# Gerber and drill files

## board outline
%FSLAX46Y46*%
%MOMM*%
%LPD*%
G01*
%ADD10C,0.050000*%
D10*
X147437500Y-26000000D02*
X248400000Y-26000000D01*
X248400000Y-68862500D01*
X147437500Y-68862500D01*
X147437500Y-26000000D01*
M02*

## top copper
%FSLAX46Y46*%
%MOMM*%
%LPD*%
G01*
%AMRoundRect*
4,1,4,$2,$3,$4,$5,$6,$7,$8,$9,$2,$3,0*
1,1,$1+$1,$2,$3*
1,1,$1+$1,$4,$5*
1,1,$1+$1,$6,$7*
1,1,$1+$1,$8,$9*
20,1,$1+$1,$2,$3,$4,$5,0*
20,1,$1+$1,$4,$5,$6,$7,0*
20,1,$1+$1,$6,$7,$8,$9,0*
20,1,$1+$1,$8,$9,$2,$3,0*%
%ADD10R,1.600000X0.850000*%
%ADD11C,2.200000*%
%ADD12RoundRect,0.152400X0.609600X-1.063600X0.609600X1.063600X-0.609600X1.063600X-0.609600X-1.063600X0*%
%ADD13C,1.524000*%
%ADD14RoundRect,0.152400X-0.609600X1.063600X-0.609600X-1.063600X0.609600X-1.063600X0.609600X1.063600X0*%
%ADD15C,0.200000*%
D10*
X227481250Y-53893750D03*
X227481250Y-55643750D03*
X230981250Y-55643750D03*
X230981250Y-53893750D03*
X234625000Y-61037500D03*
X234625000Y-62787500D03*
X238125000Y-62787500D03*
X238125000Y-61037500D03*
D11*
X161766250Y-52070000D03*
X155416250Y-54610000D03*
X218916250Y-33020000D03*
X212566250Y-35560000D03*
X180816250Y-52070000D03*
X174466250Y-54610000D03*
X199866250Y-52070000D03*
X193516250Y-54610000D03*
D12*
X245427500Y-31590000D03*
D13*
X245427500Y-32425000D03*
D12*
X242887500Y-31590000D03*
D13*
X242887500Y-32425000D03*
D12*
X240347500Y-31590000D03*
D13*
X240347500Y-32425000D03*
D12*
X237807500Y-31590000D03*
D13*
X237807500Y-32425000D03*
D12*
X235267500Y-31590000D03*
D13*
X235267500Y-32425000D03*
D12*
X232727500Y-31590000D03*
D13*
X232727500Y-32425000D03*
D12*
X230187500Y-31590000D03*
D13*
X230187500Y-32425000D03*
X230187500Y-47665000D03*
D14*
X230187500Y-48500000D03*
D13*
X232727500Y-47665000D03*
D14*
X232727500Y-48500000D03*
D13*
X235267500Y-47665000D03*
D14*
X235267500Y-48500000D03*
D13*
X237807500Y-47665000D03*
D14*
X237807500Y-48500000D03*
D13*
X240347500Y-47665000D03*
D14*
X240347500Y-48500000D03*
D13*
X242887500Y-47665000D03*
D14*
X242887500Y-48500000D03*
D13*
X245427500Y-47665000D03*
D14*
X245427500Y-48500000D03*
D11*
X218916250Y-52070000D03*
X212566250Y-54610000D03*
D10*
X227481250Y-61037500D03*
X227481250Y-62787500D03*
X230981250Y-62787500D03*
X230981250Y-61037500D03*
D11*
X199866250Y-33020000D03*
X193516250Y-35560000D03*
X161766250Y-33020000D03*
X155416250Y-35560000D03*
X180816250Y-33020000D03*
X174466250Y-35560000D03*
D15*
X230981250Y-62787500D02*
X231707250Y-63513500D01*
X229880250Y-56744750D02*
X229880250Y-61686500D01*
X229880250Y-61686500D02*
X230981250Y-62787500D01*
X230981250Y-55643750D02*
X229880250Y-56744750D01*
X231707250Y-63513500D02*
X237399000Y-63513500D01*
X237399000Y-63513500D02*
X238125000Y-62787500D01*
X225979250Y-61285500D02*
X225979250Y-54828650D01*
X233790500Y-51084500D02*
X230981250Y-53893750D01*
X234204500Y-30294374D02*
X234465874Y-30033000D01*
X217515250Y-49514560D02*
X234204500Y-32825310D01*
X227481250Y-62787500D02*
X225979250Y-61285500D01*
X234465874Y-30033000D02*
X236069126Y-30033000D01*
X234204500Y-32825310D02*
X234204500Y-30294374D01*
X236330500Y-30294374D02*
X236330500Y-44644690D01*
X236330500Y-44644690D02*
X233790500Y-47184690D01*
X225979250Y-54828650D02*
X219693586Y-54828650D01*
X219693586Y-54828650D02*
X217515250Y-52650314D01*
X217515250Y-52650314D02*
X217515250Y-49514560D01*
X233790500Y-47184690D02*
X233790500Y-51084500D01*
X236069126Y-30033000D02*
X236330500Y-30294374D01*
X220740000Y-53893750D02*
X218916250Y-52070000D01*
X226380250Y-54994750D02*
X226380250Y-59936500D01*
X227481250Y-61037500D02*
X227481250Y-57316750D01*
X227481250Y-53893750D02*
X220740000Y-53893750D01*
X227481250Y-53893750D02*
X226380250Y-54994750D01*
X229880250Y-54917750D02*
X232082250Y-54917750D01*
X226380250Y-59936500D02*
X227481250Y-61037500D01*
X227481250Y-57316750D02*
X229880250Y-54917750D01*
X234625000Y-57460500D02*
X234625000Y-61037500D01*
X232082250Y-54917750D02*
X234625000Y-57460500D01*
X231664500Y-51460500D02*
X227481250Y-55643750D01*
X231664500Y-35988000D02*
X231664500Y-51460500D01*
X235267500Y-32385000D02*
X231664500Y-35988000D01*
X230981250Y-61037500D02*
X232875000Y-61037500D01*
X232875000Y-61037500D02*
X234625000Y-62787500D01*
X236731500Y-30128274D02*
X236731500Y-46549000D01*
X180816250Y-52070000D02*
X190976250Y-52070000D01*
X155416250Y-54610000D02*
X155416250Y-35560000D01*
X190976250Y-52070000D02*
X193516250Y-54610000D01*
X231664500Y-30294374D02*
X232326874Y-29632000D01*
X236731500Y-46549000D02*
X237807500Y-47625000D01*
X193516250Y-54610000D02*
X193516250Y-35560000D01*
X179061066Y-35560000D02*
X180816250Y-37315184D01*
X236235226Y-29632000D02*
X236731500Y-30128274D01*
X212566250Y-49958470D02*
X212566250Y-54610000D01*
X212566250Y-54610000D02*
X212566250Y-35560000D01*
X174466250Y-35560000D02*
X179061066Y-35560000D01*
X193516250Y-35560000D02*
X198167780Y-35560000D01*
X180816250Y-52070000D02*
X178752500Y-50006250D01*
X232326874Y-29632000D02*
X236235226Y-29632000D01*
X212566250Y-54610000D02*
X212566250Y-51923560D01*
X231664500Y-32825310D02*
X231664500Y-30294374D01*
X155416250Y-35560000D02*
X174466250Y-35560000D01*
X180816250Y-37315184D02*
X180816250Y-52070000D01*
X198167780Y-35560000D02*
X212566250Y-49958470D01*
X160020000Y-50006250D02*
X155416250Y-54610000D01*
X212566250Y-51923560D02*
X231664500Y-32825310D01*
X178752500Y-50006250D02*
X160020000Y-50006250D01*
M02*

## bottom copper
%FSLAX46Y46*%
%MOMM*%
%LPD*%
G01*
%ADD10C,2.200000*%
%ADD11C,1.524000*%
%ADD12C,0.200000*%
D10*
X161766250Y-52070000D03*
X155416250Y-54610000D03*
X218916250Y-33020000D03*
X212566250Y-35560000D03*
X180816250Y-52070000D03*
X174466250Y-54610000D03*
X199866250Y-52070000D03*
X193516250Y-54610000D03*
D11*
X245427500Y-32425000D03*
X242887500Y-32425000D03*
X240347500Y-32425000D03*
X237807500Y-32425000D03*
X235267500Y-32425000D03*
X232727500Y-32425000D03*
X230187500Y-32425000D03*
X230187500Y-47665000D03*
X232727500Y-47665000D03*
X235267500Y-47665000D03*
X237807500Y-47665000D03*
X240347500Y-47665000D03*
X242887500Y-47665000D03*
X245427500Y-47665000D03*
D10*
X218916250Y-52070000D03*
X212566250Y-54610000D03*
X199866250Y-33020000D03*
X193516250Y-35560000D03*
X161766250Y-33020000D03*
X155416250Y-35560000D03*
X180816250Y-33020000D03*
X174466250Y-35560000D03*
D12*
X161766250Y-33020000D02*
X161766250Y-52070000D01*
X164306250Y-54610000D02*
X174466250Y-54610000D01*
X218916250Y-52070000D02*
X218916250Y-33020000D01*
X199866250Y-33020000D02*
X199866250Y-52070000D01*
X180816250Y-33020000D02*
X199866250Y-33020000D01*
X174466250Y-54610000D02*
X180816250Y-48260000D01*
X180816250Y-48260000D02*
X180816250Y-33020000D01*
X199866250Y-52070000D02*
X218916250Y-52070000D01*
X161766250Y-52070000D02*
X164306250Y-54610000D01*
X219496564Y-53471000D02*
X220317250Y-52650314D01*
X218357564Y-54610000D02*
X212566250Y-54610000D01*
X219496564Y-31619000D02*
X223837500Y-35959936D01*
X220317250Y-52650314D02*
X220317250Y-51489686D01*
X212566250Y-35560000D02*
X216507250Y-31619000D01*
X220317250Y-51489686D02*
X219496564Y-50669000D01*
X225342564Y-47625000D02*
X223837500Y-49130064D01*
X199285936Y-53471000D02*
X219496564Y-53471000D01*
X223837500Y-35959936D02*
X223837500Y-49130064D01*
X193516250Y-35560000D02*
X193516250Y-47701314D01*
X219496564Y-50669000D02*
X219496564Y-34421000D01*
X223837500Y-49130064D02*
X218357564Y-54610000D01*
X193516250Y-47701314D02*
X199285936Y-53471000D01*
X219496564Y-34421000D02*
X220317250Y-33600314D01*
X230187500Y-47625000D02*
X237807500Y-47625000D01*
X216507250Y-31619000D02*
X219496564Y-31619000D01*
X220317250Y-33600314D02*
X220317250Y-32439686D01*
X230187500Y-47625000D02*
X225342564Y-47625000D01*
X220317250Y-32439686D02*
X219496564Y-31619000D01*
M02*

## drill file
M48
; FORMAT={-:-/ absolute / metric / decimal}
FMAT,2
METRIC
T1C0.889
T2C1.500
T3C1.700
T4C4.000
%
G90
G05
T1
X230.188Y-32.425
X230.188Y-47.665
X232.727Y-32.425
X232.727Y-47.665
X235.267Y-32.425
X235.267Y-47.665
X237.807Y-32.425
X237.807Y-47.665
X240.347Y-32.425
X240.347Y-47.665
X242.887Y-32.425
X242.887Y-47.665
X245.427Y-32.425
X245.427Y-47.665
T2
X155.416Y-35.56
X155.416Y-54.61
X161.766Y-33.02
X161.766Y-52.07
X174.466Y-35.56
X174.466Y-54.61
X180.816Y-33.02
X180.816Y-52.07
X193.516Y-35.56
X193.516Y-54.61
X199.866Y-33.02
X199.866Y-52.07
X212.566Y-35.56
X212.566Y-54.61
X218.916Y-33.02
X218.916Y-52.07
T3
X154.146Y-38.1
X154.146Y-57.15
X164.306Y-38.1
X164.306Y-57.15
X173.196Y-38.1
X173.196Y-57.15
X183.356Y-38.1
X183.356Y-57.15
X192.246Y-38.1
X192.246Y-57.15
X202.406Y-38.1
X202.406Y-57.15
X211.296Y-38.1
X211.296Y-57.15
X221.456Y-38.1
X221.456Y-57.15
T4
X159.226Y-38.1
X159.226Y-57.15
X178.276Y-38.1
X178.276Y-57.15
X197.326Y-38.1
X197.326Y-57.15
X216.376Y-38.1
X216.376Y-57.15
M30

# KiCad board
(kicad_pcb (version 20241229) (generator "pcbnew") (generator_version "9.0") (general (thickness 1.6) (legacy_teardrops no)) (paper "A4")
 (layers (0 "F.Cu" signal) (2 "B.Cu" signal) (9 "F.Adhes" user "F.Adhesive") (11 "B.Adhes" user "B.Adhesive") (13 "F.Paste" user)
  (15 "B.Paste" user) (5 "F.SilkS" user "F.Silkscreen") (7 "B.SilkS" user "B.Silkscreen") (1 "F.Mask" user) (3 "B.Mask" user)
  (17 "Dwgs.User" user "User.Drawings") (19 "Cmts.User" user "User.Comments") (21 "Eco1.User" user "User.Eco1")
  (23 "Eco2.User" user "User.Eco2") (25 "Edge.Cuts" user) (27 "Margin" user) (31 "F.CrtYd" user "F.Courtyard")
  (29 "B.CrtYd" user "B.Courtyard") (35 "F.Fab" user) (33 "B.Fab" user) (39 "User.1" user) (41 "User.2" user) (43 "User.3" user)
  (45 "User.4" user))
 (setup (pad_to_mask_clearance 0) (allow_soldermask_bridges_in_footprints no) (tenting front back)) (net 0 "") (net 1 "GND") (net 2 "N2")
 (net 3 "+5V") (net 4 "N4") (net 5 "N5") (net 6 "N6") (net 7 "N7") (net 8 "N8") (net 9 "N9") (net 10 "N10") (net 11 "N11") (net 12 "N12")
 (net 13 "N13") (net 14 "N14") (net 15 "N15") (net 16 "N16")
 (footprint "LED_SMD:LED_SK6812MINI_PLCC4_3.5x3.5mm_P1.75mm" (layer "F.Cu") (at 229.23125 54.76875)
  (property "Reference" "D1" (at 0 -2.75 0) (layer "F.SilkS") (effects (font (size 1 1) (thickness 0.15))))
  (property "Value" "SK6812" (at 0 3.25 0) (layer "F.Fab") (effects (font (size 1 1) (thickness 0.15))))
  (pad "1" smd rect (at -1.75 -0.875) (size 1.6 0.85) (layers "F.Cu" "F.Mask" "F.Paste") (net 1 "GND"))
  (pad "2" smd rect (at -1.75 0.875) (size 1.6 0.85) (layers "F.Cu" "F.Mask" "F.Paste") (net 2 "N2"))
  (pad "3" smd rect (at 1.75 0.875) (size 1.6 0.85) (layers "F.Cu" "F.Mask" "F.Paste") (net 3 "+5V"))
  (pad "4" smd rect (at 1.75 -0.875) (size 1.6 0.85) (layers "F.Cu" "F.Mask" "F.Paste") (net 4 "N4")))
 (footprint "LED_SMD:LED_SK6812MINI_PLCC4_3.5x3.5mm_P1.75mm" (layer "F.Cu") (at 236.375 61.9125)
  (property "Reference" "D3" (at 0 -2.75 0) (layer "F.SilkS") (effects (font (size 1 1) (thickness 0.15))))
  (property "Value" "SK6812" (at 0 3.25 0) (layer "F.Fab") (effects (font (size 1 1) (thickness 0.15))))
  (pad "1" smd rect (at -1.75 -0.875) (size 1.6 0.85) (layers "F.Cu" "F.Mask" "F.Paste") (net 1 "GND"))
  (pad "2" smd rect (at -1.75 0.875) (size 1.6 0.85) (layers "F.Cu" "F.Mask" "F.Paste") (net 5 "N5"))
  (pad "3" smd rect (at 1.75 0.875) (size 1.6 0.85) (layers "F.Cu" "F.Mask" "F.Paste") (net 3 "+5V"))
  (pad "4" smd rect (at 1.75 -0.875) (size 1.6 0.85) (layers "F.Cu" "F.Mask" "F.Paste") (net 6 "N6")))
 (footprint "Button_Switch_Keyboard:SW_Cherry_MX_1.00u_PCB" (layer "F.Cu") (at 161.76625 52.07)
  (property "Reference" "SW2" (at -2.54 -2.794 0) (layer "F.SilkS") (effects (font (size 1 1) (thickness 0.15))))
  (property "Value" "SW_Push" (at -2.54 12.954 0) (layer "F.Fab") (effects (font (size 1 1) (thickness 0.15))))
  (pad "" np_thru_hole circle (at -7.62 5.08) (size 1.7 1.7) (drill 1.7) (layers "*.Cu" "*.Mask"))
  (pad "" np_thru_hole circle (at -2.54 5.08) (size 4 4) (drill 4) (layers "*.Cu" "*.Mask"))
  (pad "" np_thru_hole circle (at 2.54 5.08) (size 1.7 1.7) (drill 1.7) (layers "*.Cu" "*.Mask"))
  (pad "1" thru_hole circle (at 0 0) (size 2.2 2.2) (drill 1.5) (layers "*.Cu" "*.Mask") (remove_unused_layers no) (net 1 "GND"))
  (pad "2" thru_hole circle (at -6.35 2.54) (size 2.2 2.2) (drill 1.5) (layers "*.Cu" "*.Mask") (remove_unused_layers no) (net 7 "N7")))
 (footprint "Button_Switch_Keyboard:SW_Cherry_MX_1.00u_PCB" (layer "F.Cu") (at 218.91625 33.02)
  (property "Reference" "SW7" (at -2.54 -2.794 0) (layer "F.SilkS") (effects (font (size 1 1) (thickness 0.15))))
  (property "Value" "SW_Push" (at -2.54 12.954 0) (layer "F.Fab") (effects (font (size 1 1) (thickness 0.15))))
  (pad "" np_thru_hole circle (at -7.62 5.08) (size 1.7 1.7) (drill 1.7) (layers "*.Cu" "*.Mask"))
  (pad "" np_thru_hole circle (at -2.54 5.08) (size 4 4) (drill 4) (layers "*.Cu" "*.Mask"))
  (pad "" np_thru_hole circle (at 2.54 5.08) (size 1.7 1.7) (drill 1.7) (layers "*.Cu" "*.Mask"))
  (pad "1" thru_hole circle (at 0 0) (size 2.2 2.2) (drill 1.5) (layers "*.Cu" "*.Mask") (remove_unused_layers no) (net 1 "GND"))
  (pad "2" thru_hole circle (at -6.35 2.54) (size 2.2 2.2) (drill 1.5) (layers "*.Cu" "*.Mask") (remove_unused_layers no) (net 7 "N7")))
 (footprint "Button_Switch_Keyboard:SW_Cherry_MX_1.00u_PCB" (layer "F.Cu") (at 180.81625 52.07)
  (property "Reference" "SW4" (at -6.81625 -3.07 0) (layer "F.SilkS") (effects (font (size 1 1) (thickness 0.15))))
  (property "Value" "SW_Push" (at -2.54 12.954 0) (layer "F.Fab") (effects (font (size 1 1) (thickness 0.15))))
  (pad "" np_thru_hole circle (at -7.62 5.08) (size 1.7 1.7) (drill 1.7) (layers "*.Cu" "*.Mask"))
  (pad "" np_thru_hole circle (at -2.54 5.08) (size 4 4) (drill 4) (layers "*.Cu" "*.Mask"))
  (pad "" np_thru_hole circle (at 2.54 5.08) (size 1.7 1.7) (drill 1.7) (layers "*.Cu" "*.Mask"))
  (pad "1" thru_hole circle (at 0 0) (size 2.2 2.2) (drill 1.5) (layers "*.Cu" "*.Mask") (remove_unused_layers no) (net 7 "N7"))
  (pad "2" thru_hole circle (at -6.35 2.54) (size 2.2 2.2) (drill 1.5) (layers "*.Cu" "*.Mask") (remove_unused_layers no) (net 1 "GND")))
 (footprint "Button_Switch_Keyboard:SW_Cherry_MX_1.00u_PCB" (layer "F.Cu") (at 199.86625 52.07)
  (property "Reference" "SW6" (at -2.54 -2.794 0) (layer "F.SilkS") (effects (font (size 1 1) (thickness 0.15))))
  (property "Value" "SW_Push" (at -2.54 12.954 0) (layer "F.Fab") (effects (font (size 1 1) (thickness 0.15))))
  (pad "" np_thru_hole circle (at -7.62 5.08) (size 1.7 1.7) (drill 1.7) (layers "*.Cu" "*.Mask"))
  (pad "" np_thru_hole circle (at -2.54 5.08) (size 4 4) (drill 4) (layers "*.Cu" "*.Mask"))
  (pad "" np_thru_hole circle (at 2.54 5.08) (size 1.7 1.7) (drill 1.7) (layers "*.Cu" "*.Mask"))
  (pad "1" thru_hole circle (at 0 0) (size 2.2 2.2) (drill 1.5) (layers "*.Cu" "*.Mask") (remove_unused_layers no) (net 1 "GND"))
  (pad "2" thru_hole circle (at -6.35 2.54) (size 2.2 2.2) (drill 1.5) (layers "*.Cu" "*.Mask") (remove_unused_layers no) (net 7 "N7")))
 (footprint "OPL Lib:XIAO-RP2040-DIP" (layer "F.Cu") (at 237.8075 40.045 -90)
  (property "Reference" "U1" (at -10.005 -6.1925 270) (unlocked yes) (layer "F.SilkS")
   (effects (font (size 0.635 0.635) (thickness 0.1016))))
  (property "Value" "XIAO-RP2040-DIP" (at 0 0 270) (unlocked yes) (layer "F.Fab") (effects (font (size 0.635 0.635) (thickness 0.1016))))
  (pad "1" smd roundrect (at -8.455 -7.62 90) (size 2.432 1.524) (layers "F.Cu" "F.Mask") (roundrect_rratio 0.1) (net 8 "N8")
   (thermal_bridge_angle 45))
  (pad "1" thru_hole circle (at -7.62 -7.62 90) (size 1.524 1.524) (drill 0.889) (layers "*.Cu" "*.Mask") (remove_unused_layers no)
   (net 8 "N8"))
  (pad "2" smd roundrect (at -8.455 -5.08 90) (size 2.432 1.524) (layers "F.Cu" "F.Mask") (roundrect_rratio 0.1) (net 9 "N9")
   (thermal_bridge_angle 45))
  (pad "2" thru_hole circle (at -7.62 -5.08 90) (size 1.524 1.524) (drill 0.889) (layers "*.Cu" "*.Mask") (remove_unused_layers no)
   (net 9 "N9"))
  (pad "3" smd roundrect (at -8.455 -2.54 90) (size 2.432 1.524) (layers "F.Cu" "F.Mask") (roundrect_rratio 0.1) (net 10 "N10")
   (thermal_bridge_angle 45))
  (pad "3" thru_hole circle (at -7.62 -2.54 90) (size 1.524 1.524) (drill 0.889) (layers "*.Cu" "*.Mask") (remove_unused_layers no)
   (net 10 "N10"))
  (pad "4" smd roundrect (at -8.455 0 90) (size 2.432 1.524) (layers "F.Cu" "F.Mask") (roundrect_rratio 0.1) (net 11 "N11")
   (thermal_bridge_angle 45))
  (pad "4" thru_hole circle (at -7.62 0 90) (size 1.524 1.524) (drill 0.889) (layers "*.Cu" "*.Mask") (remove_unused_layers no)
   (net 11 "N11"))
  (pad "5" smd roundrect (at -8.455 2.54 90) (size 2.432 1.524) (layers "F.Cu" "F.Mask") (roundrect_rratio 0.1) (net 2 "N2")
   (thermal_bridge_angle 45))
  (pad "5" thru_hole circle (at -7.62 2.54 90) (size 1.524 1.524) (drill 0.889) (layers "*.Cu" "*.Mask") (remove_unused_layers no)
   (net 2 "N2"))
  (pad "6" smd roundrect (at -8.455 5.08 90) (size 2.432 1.524) (layers "F.Cu" "F.Mask") (roundrect_rratio 0.1) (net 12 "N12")
   (thermal_bridge_angle 45))
  (pad "6" thru_hole circle (at -7.62 5.08 90) (size 1.524 1.524) (drill 0.889) (layers "*.Cu" "*.Mask") (remove_unused_layers no)
   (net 12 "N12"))
  (pad "7" smd roundrect (at -8.455 7.62 90) (size 2.432 1.524) (layers "F.Cu" "F.Mask") (roundrect_rratio 0.1) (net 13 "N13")
   (thermal_bridge_angle 45))
  (pad "7" thru_hole circle (at -7.62 7.62 90) (size 1.524 1.524) (drill 0.889) (layers "*.Cu" "*.Mask") (remove_unused_layers no)
   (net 13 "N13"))
  (pad "8" thru_hole circle (at 7.62 7.62 270) (size 1.524 1.524) (drill 0.889) (layers "*.Cu" "*.Mask") (remove_unused_layers no)
   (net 7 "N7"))
  (pad "8" smd roundrect (at 8.455 7.62 270) (size 2.432 1.524) (layers "F.Cu" "F.Mask") (roundrect_rratio 0.1) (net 7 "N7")
   (thermal_bridge_angle 45))
  (pad "9" thru_hole circle (at 7.62 5.08 270) (size 1.524 1.524) (drill 0.889) (layers "*.Cu" "*.Mask") (remove_unused_layers no)
   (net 7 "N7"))
  (pad "9" smd roundrect (at 8.455 5.08 270) (size 2.432 1.524) (layers "F.Cu" "F.Mask") (roundrect_rratio 0.1) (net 7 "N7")
   (thermal_bridge_angle 45))
  (pad "10" thru_hole circle (at 7.62 2.54 270) (size 1.524 1.524) (drill 0.889) (layers "*.Cu" "*.Mask") (remove_unused_layers no)
   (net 7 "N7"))
  (pad "10" smd roundrect (at 8.455 2.54 270) (size 2.432 1.524) (layers "F.Cu" "F.Mask") (roundrect_rratio 0.1) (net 7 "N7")
   (thermal_bridge_angle 45))
  (pad "11" thru_hole circle (at 7.62 0 270) (size 1.524 1.524) (drill 0.889) (layers "*.Cu" "*.Mask") (remove_unused_layers no)
   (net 7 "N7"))
  (pad "11" smd roundrect (at 8.455 0 270) (size 2.432 1.524) (layers "F.Cu" "F.Mask") (roundrect_rratio 0.1) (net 7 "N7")
   (thermal_bridge_angle 45))
  (pad "12" thru_hole circle (at 7.62 -2.54 270) (size 1.524 1.524) (drill 0.889) (layers "*.Cu" "*.Mask") (remove_unused_layers no)
   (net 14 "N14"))
  (pad "12" smd roundrect (at 8.455 -2.54 270) (size 2.432 1.524) (layers "F.Cu" "F.Mask") (roundrect_rratio 0.1) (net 14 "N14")
   (thermal_bridge_angle 45))
  (pad "13" thru_hole circle (at 7.62 -5.08 270) (size 1.524 1.524) (drill 0.889) (layers "*.Cu" "*.Mask") (remove_unused_layers no)
   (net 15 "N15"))
  (pad "13" smd roundrect (at 8.455 -5.08 270) (size 2.432 1.524) (layers "F.Cu" "F.Mask") (roundrect_rratio 0.1) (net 15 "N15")
   (thermal_bridge_angle 45))
  (pad "14" thru_hole circle (at 7.62 -7.62 270) (size 1.524 1.524) (drill 0.889) (layers "*.Cu" "*.Mask") (remove_unused_layers no)
   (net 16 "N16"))
  (pad "14" smd roundrect (at 8.455 -7.62 270) (size 2.432 1.524) (layers "F.Cu" "F.Mask") (roundrect_rratio 0.1) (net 16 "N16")
   (thermal_bridge_angle 45)))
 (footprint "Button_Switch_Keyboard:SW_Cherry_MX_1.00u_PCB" (layer "F.Cu") (at 218.91625 52.07)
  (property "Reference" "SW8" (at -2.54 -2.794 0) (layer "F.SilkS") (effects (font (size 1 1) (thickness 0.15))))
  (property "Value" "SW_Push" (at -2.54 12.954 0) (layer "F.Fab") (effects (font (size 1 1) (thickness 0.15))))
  (pad "" np_thru_hole circle (at -7.62 5.08) (size 1.7 1.7) (drill 1.7) (layers "*.Cu" "*.Mask"))
  (pad "" np_thru_hole circle (at -2.54 5.08) (size 4 4) (drill 4) (layers "*.Cu" "*.Mask"))
  (pad "" np_thru_hole circle (at 2.54 5.08) (size 1.7 1.7) (drill 1.7) (layers "*.Cu" "*.Mask"))
  (pad "1" thru_hole circle (at 0 0) (size 2.2 2.2) (drill 1.5) (layers "*.Cu" "*.Mask") (remove_unused_layers no) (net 1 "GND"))
  (pad "2" thru_hole circle (at -6.35 2.54) (size 2.2 2.2) (drill 1.5) (layers "*.Cu" "*.Mask") (remove_unused_layers no) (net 7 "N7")))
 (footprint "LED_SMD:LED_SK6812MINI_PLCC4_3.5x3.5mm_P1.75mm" (layer "F.Cu") (at 229.23125 61.9125)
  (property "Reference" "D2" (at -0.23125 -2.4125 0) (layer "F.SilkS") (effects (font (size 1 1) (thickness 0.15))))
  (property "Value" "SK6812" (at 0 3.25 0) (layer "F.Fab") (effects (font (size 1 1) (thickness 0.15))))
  (pad "1" smd rect (at -1.75 -0.875) (size 1.6 0.85) (layers "F.Cu" "F.Mask" "F.Paste") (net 1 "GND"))
  (pad "2" smd rect (at -1.75 0.875) (size 1.6 0.85) (layers "F.Cu" "F.Mask" "F.Paste") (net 4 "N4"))
  (pad "3" smd rect (at 1.75 0.875) (size 1.6 0.85) (layers "F.Cu" "F.Mask" "F.Paste") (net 3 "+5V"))
  (pad "4" smd rect (at 1.75 -0.875) (size 1.6 0.85) (layers "F.Cu" "F.Mask" "F.Paste") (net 5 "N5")))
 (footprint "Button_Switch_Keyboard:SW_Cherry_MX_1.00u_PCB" (layer "F.Cu") (at 199.86625 33.02)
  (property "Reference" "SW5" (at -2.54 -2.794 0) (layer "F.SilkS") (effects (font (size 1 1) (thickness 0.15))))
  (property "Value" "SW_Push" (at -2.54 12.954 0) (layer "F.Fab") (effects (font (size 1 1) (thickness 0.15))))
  (pad "" np_thru_hole circle (at -7.62 5.08) (size 1.7 1.7) (drill 1.7) (layers "*.Cu" "*.Mask"))
  (pad "" np_thru_hole circle (at -2.54 5.08) (size 4 4) (drill 4) (layers "*.Cu" "*.Mask"))
  (pad "" np_thru_hole circle (at 2.54 5.08) (size 1.7 1.7) (drill 1.7) (layers "*.Cu" "*.Mask"))
  (pad "1" thru_hole circle (at 0 0) (size 2.2 2.2) (drill 1.5) (layers "*.Cu" "*.Mask") (remove_unused_layers no) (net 1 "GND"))
  (pad "2" thru_hole circle (at -6.35 2.54) (size 2.2 2.2) (drill 1.5) (layers "*.Cu" "*.Mask") (remove_unused_layers no) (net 7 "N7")))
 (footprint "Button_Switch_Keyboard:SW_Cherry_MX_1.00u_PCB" (layer "F.Cu") (at 161.76625 33.02)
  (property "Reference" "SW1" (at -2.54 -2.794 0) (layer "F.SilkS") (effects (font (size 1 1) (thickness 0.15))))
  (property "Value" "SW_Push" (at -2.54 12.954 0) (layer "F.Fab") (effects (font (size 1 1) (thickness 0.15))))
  (pad "" np_thru_hole circle (at -7.62 5.08) (size 1.7 1.7) (drill 1.7) (layers "*.Cu" "*.Mask"))
  (pad "" np_thru_hole circle (at -2.54 5.08) (size 4 4) (drill 4) (layers "*.Cu" "*.Mask"))
  (pad "" np_thru_hole circle (at 2.54 5.08) (size 1.7 1.7) (drill 1.7) (layers "*.Cu" "*.Mask"))
  (pad "1" thru_hole circle (at 0 0) (size 2.2 2.2) (drill 1.5) (layers "*.Cu" "*.Mask") (remove_unused_layers no) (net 1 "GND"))
  (pad "2" thru_hole circle (at -6.35 2.54) (size 2.2 2.2) (drill 1.5) (layers "*.Cu" "*.Mask") (remove_unused_layers no) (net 7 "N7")))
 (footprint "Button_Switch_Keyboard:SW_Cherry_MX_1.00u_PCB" (layer "F.Cu") (at 180.81625 33.02)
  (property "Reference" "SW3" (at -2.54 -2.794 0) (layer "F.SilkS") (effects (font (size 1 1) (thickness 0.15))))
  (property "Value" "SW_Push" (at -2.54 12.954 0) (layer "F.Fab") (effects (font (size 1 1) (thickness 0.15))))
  (pad "" np_thru_hole circle (at -7.62 5.08) (size 1.7 1.7) (drill 1.7) (layers "*.Cu" "*.Mask"))
  (pad "" np_thru_hole circle (at -2.54 5.08) (size 4 4) (drill 4) (layers "*.Cu" "*.Mask"))
  (pad "" np_thru_hole circle (at 2.54 5.08) (size 1.7 1.7) (drill 1.7) (layers "*.Cu" "*.Mask"))
  (pad "1" thru_hole circle (at 0 0) (size 2.2 2.2) (drill 1.5) (layers "*.Cu" "*.Mask") (remove_unused_layers no) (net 1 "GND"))
  (pad "2" thru_hole circle (at -6.35 2.54) (size 2.2 2.2) (drill 1.5) (layers "*.Cu" "*.Mask") (remove_unused_layers no) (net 7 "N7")))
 (gr_rect (start 147.4375 26) (end 248.4 68.8625) (stroke (width 0.05) (type solid)) (fill no) (layer "Edge.Cuts"))
 (segment (start 230.98125 62.7875) (end 231.70725 63.5135) (width 0.2) (layer "F.Cu") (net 3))
 (segment (start 229.88025 56.74475) (end 229.88025 61.6865) (width 0.2) (layer "F.Cu") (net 3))
 (segment (start 229.88025 61.6865) (end 230.98125 62.7875) (width 0.2) (layer "F.Cu") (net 3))
 (segment (start 230.98125 55.64375) (end 229.88025 56.74475) (width 0.2) (layer "F.Cu") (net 3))
 (segment (start 231.70725 63.5135) (end 237.399 63.5135) (width 0.2) (layer "F.Cu") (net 3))
 (segment (start 237.399 63.5135) (end 238.125 62.7875) (width 0.2) (layer "F.Cu") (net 3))
 (segment (start 225.97925 61.2855) (end 225.97925 54.82865) (width 0.2) (layer "F.Cu") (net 4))
 (segment (start 233.7905 51.0845) (end 230.98125 53.89375) (width 0.2) (layer "F.Cu") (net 4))
 (segment (start 234.2045 30.294374) (end 234.465874 30.033) (width 0.2) (layer "F.Cu") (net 4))
 (segment (start 217.51525 49.51456) (end 234.2045 32.82531) (width 0.2) (layer "F.Cu") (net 4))
 (segment (start 227.48125 62.7875) (end 225.97925 61.2855) (width 0.2) (layer "F.Cu") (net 4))
 (segment (start 234.465874 30.033) (end 236.069126 30.033) (width 0.2) (layer "F.Cu") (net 4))
 (segment (start 234.2045 32.82531) (end 234.2045 30.294374) (width 0.2) (layer "F.Cu") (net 4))
 (segment (start 236.3305 30.294374) (end 236.3305 44.64469) (width 0.2) (layer "F.Cu") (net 4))
 (segment (start 236.3305 44.64469) (end 233.7905 47.18469) (width 0.2) (layer "F.Cu") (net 4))
 (segment (start 225.97925 54.82865) (end 219.693586 54.82865) (width 0.2) (layer "F.Cu") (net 4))
 (segment (start 219.693586 54.82865) (end 217.51525 52.650314) (width 0.2) (layer "F.Cu") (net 4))
 (segment (start 217.51525 52.650314) (end 217.51525 49.51456) (width 0.2) (layer "F.Cu") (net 4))
 (segment (start 233.7905 47.18469) (end 233.7905 51.0845) (width 0.2) (layer "F.Cu") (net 4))
 (segment (start 236.069126 30.033) (end 236.3305 30.294374) (width 0.2) (layer "F.Cu") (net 4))
 (segment (start 220.74 53.89375) (end 218.91625 52.07) (width 0.2) (layer "F.Cu") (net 1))
 (segment (start 226.38025 54.99475) (end 226.38025 59.9365) (width 0.2) (layer "F.Cu") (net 1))
 (segment (start 227.48125 61.0375) (end 227.48125 57.31675) (width 0.2) (layer "F.Cu") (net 1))
 (segment (start 227.48125 53.89375) (end 220.74 53.89375) (width 0.2) (layer "F.Cu") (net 1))
 (segment (start 227.48125 53.89375) (end 226.38025 54.99475) (width 0.2) (layer "F.Cu") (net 1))
 (segment (start 229.88025 54.91775) (end 232.08225 54.91775) (width 0.2) (layer "F.Cu") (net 1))
 (segment (start 226.38025 59.9365) (end 227.48125 61.0375) (width 0.2) (layer "F.Cu") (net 1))
 (segment (start 227.48125 57.31675) (end 229.88025 54.91775) (width 0.2) (layer "F.Cu") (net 1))
 (segment (start 234.625 57.4605) (end 234.625 61.0375) (width 0.2) (layer "F.Cu") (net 1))
 (segment (start 232.08225 54.91775) (end 234.625 57.4605) (width 0.2) (layer "F.Cu") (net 1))
 (segment (start 161.76625 33.02) (end 161.76625 52.07) (width 0.2) (layer "B.Cu") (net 1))
 (segment (start 164.30625 54.61) (end 174.46625 54.61) (width 0.2) (layer "B.Cu") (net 1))
 (segment (start 218.91625 52.07) (end 218.91625 33.02) (width 0.2) (layer "B.Cu") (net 1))
 (segment (start 199.86625 33.02) (end 199.86625 52.07) (width 0.2) (layer "B.Cu") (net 1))
 (segment (start 180.81625 33.02) (end 199.86625 33.02) (width 0.2) (layer "B.Cu") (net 1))
 (segment (start 174.46625 54.61) (end 180.81625 48.26) (width 0.2) (layer "B.Cu") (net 1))
 (segment (start 180.81625 48.26) (end 180.81625 33.02) (width 0.2) (layer "B.Cu") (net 1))
 (segment (start 199.86625 52.07) (end 218.91625 52.07) (width 0.2) (layer "B.Cu") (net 1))
 (segment (start 161.76625 52.07) (end 164.30625 54.61) (width 0.2) (layer "B.Cu") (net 1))
 (segment (start 231.6645 51.4605) (end 227.48125 55.64375) (width 0.2) (layer "F.Cu") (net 2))
 (segment (start 231.6645 35.988) (end 231.6645 51.4605) (width 0.2) (layer "F.Cu") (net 2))
 (segment (start 235.2675 32.385) (end 231.6645 35.988) (width 0.2) (layer "F.Cu") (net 2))
 (segment (start 230.98125 61.0375) (end 232.875 61.0375) (width 0.2) (layer "F.Cu") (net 5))
 (segment (start 232.875 61.0375) (end 234.625 62.7875) (width 0.2) (layer "F.Cu") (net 5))
 (segment (start 236.7315 30.128274) (end 236.7315 46.549) (width 0.2) (layer "F.Cu") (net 7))
 (segment (start 180.81625 52.07) (end 190.97625 52.07) (width 0.2) (layer "F.Cu") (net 7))
 (segment (start 155.41625 54.61) (end 155.41625 35.56) (width 0.2) (layer "F.Cu") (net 7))
 (segment (start 190.97625 52.07) (end 193.51625 54.61) (width 0.2) (layer "F.Cu") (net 7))
 (segment (start 231.6645 30.294374) (end 232.326874 29.632) (width 0.2) (layer "F.Cu") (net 7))
 (segment (start 236.7315 46.549) (end 237.8075 47.625) (width 0.2) (layer "F.Cu") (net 7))
 (segment (start 193.51625 54.61) (end 193.51625 35.56) (width 0.2) (layer "F.Cu") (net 7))
 (segment (start 179.061066 35.56) (end 180.81625 37.315184) (width 0.2) (layer "F.Cu") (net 7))
 (segment (start 236.235226 29.632) (end 236.7315 30.128274) (width 0.2) (layer "F.Cu") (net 7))
 (segment (start 212.56625 49.95847) (end 212.56625 54.61) (width 0.2) (layer "F.Cu") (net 7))
 (segment (start 212.56625 54.61) (end 212.56625 35.56) (width 0.2) (layer "F.Cu") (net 7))
 (segment (start 174.46625 35.56) (end 179.061066 35.56) (width 0.2) (layer "F.Cu") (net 7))
 (segment (start 193.51625 35.56) (end 198.16778 35.56) (width 0.2) (layer "F.Cu") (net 7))
 (segment (start 180.81625 52.07) (end 178.7525 50.00625) (width 0.2) (layer "F.Cu") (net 7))
 (segment (start 232.326874 29.632) (end 236.235226 29.632) (width 0.2) (layer "F.Cu") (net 7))
 (segment (start 212.56625 54.61) (end 212.56625 51.92356) (width 0.2) (layer "F.Cu") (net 7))
 (segment (start 231.6645 32.82531) (end 231.6645 30.294374) (width 0.2) (layer "F.Cu") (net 7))
 (segment (start 155.41625 35.56) (end 174.46625 35.56) (width 0.2) (layer "F.Cu") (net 7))
 (segment (start 180.81625 37.315184) (end 180.81625 52.07) (width 0.2) (layer "F.Cu") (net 7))
 (segment (start 198.16778 35.56) (end 212.56625 49.95847) (width 0.2) (layer "F.Cu") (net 7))
 (segment (start 160.02 50.00625) (end 155.41625 54.61) (width 0.2) (layer "F.Cu") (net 7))
 (segment (start 212.56625 51.92356) (end 231.6645 32.82531) (width 0.2) (layer "F.Cu") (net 7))
 (segment (start 178.7525 50.00625) (end 160.02 50.00625) (width 0.2) (layer "F.Cu") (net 7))
 (segment (start 219.496564 53.471) (end 220.31725 52.650314) (width 0.2) (layer "B.Cu") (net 7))
 (segment (start 218.357564 54.61) (end 212.56625 54.61) (width 0.2) (layer "B.Cu") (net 7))
 (segment (start 219.496564 31.619) (end 223.8375 35.959936) (width 0.2) (layer "B.Cu") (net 7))
 (segment (start 220.31725 52.650314) (end 220.31725 51.489686) (width 0.2) (layer "B.Cu") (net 7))
 (segment (start 212.56625 35.56) (end 216.50725 31.619) (width 0.2) (layer "B.Cu") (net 7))
 (segment (start 220.31725 51.489686) (end 219.496564 50.669) (width 0.2) (layer "B.Cu") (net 7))
 (segment (start 225.342564 47.625) (end 223.8375 49.130064) (width 0.2) (layer "B.Cu") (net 7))
 (segment (start 199.285936 53.471) (end 219.496564 53.471) (width 0.2) (layer "B.Cu") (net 7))
 (segment (start 223.8375 35.959936) (end 223.8375 49.130064) (width 0.2) (layer "B.Cu") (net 7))
 (segment (start 193.51625 35.56) (end 193.51625 47.701314) (width 0.2) (layer "B.Cu") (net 7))
 (segment (start 219.496564 50.669) (end 219.496564 34.421) (width 0.2) (layer "B.Cu") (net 7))
 (segment (start 223.8375 49.130064) (end 218.357564 54.61) (width 0.2) (layer "B.Cu") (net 7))
 (segment (start 193.51625 47.701314) (end 199.285936 53.471) (width 0.2) (layer "B.Cu") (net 7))
 (segment (start 219.496564 34.421) (end 220.31725 33.600314) (width 0.2) (layer "B.Cu") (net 7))
 (segment (start 230.1875 47.625) (end 237.8075 47.625) (width 0.2) (layer "B.Cu") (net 7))
 (segment (start 216.50725 31.619) (end 219.496564 31.619) (width 0.2) (layer "B.Cu") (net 7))
 (segment (start 220.31725 33.600314) (end 220.31725 32.439686) (width 0.2) (layer "B.Cu") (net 7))
 (segment (start 230.1875 47.625) (end 225.342564 47.625) (width 0.2) (layer "B.Cu") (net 7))
 (segment (start 220.31725 32.439686) (end 219.496564 31.619) (width 0.2) (layer "B.Cu") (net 7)))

